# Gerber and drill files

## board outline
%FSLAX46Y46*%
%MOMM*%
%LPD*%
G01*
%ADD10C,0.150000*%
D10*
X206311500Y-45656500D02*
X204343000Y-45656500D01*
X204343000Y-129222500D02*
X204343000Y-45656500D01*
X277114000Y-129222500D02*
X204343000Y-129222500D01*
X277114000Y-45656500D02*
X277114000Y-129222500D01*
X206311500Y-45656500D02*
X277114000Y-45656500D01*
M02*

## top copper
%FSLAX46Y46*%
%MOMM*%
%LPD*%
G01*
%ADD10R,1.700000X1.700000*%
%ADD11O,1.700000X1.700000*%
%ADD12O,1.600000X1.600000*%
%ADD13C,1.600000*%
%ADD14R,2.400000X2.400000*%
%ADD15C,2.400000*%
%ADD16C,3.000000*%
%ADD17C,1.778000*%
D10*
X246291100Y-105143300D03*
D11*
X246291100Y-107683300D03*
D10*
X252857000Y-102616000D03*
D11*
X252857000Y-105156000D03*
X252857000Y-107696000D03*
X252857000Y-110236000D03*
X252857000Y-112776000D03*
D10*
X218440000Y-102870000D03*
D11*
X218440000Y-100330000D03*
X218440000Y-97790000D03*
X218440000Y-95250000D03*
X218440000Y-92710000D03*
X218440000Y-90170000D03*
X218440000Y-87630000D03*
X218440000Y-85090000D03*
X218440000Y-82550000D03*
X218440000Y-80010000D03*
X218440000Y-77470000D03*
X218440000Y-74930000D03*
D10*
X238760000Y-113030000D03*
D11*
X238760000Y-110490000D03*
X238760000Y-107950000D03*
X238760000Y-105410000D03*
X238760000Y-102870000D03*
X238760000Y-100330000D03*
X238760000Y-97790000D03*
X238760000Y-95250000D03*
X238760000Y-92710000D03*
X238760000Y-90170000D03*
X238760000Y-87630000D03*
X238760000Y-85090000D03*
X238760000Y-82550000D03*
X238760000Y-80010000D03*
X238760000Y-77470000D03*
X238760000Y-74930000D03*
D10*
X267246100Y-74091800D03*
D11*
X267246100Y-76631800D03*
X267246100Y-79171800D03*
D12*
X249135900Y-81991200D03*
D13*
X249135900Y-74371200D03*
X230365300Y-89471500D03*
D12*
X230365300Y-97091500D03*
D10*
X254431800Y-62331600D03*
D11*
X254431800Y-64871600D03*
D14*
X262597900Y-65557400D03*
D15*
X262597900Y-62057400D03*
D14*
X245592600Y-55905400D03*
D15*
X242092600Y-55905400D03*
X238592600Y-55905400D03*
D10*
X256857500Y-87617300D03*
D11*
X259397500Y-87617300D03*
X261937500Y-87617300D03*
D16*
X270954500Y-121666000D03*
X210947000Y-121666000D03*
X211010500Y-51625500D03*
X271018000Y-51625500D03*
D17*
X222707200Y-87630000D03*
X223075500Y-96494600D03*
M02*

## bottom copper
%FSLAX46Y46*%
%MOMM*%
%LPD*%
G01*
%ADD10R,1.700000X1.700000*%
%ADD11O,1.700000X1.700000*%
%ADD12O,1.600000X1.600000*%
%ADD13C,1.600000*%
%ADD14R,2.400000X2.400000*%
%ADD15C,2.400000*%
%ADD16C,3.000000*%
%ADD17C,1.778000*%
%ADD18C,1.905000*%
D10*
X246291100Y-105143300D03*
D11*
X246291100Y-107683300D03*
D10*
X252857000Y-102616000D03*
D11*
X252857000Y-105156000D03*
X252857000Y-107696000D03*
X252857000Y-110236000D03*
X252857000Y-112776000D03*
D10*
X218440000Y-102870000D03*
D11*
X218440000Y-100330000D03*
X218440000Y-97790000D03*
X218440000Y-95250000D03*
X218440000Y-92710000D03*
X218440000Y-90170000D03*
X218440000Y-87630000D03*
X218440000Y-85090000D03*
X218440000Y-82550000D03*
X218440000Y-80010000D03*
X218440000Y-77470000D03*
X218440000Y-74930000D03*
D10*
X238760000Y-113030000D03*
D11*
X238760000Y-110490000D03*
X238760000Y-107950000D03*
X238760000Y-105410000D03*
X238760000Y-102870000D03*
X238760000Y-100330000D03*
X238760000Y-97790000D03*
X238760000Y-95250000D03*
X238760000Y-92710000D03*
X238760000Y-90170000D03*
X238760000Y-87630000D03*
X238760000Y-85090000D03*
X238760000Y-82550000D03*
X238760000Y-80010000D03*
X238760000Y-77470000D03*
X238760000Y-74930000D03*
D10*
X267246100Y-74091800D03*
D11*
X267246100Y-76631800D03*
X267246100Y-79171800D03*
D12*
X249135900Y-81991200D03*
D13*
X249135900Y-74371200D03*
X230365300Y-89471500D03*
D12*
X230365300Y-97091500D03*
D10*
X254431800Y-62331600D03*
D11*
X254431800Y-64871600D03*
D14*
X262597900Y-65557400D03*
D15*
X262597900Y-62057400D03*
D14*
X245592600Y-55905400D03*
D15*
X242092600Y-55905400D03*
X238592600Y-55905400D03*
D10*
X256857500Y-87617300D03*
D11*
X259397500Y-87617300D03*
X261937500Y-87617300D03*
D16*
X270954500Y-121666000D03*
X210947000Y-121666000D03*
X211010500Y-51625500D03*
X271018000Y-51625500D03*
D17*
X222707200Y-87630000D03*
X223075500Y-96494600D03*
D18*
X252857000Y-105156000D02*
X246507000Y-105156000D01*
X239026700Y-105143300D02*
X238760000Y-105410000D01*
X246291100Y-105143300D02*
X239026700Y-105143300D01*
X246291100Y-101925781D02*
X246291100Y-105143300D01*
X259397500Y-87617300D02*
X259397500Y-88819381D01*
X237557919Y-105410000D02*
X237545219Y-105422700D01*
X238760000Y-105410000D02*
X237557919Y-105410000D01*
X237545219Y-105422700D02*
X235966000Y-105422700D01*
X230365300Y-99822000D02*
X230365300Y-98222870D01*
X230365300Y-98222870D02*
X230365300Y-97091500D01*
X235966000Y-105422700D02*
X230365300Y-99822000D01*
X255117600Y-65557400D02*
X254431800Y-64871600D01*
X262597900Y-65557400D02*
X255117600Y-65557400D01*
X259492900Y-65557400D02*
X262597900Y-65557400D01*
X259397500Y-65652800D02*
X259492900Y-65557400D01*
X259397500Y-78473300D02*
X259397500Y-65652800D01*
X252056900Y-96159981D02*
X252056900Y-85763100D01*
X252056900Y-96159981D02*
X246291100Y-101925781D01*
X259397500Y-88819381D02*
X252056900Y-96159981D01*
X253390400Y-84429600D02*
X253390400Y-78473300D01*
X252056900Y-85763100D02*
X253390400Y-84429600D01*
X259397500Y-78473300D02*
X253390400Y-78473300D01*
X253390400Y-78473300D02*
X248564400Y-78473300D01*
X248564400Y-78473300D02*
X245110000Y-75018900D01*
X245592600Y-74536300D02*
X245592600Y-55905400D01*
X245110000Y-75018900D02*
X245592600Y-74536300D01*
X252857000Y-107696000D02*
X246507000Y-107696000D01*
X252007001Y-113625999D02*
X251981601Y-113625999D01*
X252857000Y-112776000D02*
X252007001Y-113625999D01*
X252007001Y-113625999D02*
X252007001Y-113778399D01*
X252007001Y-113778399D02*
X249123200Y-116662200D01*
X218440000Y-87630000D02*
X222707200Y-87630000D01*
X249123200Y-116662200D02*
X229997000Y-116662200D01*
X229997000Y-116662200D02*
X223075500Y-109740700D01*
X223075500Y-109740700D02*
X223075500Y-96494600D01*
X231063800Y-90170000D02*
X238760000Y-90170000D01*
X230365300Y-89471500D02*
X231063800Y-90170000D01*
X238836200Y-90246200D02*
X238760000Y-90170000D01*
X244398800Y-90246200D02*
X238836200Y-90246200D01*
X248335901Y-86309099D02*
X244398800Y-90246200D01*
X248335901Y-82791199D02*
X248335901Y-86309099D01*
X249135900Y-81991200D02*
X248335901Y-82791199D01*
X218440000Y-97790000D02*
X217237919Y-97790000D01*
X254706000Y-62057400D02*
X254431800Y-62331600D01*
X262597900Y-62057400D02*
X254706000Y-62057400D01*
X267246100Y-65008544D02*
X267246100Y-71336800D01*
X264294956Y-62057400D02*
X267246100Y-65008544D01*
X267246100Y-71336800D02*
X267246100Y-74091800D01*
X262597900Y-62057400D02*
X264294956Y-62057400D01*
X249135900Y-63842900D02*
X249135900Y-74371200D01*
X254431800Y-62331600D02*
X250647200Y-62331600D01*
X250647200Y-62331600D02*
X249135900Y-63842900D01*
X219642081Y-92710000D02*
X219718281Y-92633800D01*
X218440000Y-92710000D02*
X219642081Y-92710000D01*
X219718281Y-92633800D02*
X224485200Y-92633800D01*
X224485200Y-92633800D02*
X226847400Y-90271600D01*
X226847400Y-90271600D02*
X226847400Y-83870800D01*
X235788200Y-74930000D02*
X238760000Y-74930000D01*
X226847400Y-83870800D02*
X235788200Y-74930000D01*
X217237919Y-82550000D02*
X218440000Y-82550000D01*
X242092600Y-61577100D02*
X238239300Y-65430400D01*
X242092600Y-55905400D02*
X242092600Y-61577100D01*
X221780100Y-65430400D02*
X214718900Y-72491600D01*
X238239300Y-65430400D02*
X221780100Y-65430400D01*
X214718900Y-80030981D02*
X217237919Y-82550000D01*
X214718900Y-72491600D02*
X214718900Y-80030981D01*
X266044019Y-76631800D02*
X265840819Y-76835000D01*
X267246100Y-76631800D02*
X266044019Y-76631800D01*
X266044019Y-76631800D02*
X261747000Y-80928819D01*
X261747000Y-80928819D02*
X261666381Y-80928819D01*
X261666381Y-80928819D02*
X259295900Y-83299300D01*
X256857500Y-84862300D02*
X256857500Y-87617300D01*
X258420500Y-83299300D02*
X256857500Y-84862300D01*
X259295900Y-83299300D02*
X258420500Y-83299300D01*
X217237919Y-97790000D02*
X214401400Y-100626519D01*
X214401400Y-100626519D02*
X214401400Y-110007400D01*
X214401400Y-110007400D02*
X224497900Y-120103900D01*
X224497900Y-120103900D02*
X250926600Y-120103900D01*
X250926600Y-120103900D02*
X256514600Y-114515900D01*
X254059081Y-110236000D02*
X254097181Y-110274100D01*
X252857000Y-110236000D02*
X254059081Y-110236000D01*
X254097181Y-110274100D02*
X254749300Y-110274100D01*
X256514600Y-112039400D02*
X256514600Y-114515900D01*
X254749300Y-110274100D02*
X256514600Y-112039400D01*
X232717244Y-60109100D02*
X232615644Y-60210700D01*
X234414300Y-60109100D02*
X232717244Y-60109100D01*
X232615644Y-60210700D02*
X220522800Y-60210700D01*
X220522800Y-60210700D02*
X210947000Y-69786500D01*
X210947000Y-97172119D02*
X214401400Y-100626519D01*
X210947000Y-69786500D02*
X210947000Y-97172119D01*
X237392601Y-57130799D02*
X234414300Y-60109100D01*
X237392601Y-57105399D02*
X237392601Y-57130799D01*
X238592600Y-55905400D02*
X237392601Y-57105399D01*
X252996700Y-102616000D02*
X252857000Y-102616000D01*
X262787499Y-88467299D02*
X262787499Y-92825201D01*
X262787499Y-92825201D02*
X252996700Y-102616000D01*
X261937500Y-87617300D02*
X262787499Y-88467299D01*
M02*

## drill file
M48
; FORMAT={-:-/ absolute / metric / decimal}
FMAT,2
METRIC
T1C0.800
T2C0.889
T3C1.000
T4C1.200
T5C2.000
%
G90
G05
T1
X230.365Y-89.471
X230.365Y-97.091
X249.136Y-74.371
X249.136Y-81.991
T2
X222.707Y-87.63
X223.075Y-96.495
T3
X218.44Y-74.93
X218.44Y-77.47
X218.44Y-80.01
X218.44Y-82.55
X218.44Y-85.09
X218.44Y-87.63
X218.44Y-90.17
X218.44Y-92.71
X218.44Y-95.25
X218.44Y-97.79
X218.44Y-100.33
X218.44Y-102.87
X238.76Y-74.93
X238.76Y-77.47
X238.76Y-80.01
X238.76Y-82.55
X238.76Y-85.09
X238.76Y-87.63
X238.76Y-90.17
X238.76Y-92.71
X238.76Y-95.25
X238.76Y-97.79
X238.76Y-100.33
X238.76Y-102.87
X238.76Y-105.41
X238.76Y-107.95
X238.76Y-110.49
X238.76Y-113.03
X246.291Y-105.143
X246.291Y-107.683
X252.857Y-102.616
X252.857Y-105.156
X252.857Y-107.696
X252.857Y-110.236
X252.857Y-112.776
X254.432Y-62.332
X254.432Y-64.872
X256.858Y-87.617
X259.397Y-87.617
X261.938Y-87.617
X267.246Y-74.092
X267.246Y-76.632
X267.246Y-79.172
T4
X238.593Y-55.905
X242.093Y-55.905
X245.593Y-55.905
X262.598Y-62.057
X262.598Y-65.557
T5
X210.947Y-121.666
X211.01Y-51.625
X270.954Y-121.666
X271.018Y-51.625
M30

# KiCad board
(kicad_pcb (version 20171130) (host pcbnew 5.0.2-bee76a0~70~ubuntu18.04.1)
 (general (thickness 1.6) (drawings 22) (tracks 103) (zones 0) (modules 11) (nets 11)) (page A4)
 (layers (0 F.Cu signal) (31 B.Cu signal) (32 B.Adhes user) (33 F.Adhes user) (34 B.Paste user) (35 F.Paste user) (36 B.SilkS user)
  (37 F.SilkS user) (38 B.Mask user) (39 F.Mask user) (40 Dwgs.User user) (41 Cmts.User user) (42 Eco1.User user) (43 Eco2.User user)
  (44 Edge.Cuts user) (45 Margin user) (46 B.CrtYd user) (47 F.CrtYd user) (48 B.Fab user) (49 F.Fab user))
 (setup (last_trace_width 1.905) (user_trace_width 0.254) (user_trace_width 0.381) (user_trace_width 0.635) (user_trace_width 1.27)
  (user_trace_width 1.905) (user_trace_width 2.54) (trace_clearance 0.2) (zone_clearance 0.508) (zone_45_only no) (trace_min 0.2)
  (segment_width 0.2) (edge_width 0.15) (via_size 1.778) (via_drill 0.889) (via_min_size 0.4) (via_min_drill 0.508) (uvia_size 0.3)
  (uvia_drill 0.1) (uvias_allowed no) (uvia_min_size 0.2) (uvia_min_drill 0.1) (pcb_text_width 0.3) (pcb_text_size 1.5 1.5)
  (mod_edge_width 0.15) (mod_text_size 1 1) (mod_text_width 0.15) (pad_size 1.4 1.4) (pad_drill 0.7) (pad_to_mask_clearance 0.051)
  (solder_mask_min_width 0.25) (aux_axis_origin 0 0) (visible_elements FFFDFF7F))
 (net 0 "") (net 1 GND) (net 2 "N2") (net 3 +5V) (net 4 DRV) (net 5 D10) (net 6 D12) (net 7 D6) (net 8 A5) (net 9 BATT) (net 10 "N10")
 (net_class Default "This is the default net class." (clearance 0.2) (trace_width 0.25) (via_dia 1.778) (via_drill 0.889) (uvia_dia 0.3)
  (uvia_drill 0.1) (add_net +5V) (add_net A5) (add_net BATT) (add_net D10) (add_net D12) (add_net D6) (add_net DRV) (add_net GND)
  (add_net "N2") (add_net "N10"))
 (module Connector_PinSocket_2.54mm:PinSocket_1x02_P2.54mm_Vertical (layer F.Cu) (at 246.2911 105.1433)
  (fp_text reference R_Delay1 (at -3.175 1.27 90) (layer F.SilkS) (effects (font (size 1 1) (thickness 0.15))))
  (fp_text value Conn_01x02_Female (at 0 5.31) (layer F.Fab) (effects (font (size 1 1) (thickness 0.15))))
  (pad 1 thru_hole rect (at 0 0) (size 1.7 1.7) (drill 1) (layers *.Cu *.Mask) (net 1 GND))
  (pad 2 thru_hole oval (at 0 2.54) (size 1.7 1.7) (drill 1) (layers *.Cu *.Mask) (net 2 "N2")))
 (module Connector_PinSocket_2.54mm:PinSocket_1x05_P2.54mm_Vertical (layer F.Cu) (at 252.857 102.616)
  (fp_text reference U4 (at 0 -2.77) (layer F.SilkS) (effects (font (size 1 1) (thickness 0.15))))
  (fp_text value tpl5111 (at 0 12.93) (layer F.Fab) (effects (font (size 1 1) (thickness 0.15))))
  (pad 1 thru_hole rect (at 0 0) (size 1.7 1.7) (drill 1) (layers *.Cu *.Mask) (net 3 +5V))
  (pad 2 thru_hole oval (at 0 2.54) (size 1.7 1.7) (drill 1) (layers *.Cu *.Mask) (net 1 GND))
  (pad 3 thru_hole oval (at 0 5.08) (size 1.7 1.7) (drill 1) (layers *.Cu *.Mask) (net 2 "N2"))
  (pad 4 thru_hole oval (at 0 7.62) (size 1.7 1.7) (drill 1) (layers *.Cu *.Mask) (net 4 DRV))
  (pad 5 thru_hole oval (at 0 10.16) (size 1.7 1.7) (drill 1) (layers *.Cu *.Mask) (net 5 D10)))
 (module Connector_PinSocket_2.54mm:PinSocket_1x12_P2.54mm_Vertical (layer F.Cu) (at 218.44 102.87 180)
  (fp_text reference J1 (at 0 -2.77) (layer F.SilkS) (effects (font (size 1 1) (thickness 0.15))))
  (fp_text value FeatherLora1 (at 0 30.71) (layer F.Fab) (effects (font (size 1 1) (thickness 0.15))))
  (pad 1 thru_hole rect (at 0 0 180) (size 1.7 1.7) (drill 1) (layers *.Cu *.Mask))
  (pad 2 thru_hole oval (at 0 2.54 180) (size 1.7 1.7) (drill 1) (layers *.Cu *.Mask))
  (pad 3 thru_hole oval (at 0 5.08 180) (size 1.7 1.7) (drill 1) (layers *.Cu *.Mask) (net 4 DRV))
  (pad 4 thru_hole oval (at 0 7.62 180) (size 1.7 1.7) (drill 1) (layers *.Cu *.Mask))
  (pad 5 thru_hole oval (at 0 10.16 180) (size 1.7 1.7) (drill 1) (layers *.Cu *.Mask) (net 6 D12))
  (pad 6 thru_hole oval (at 0 12.7 180) (size 1.7 1.7) (drill 1) (layers *.Cu *.Mask))
  (pad 7 thru_hole oval (at 0 15.24 180) (size 1.7 1.7) (drill 1) (layers *.Cu *.Mask) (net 5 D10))
  (pad 8 thru_hole oval (at 0 17.78 180) (size 1.7 1.7) (drill 1) (layers *.Cu *.Mask))
  (pad 9 thru_hole oval (at 0 20.32 180) (size 1.7 1.7) (drill 1) (layers *.Cu *.Mask) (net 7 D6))
  (pad 10 thru_hole oval (at 0 22.86 180) (size 1.7 1.7) (drill 1) (layers *.Cu *.Mask))
  (pad 11 thru_hole oval (at 0 25.4 180) (size 1.7 1.7) (drill 1) (layers *.Cu *.Mask))
  (pad 12 thru_hole oval (at 0 27.94 180) (size 1.7 1.7) (drill 1) (layers *.Cu *.Mask)))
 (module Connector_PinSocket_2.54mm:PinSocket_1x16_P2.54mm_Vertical (layer F.Cu) (at 238.76 113.03 180)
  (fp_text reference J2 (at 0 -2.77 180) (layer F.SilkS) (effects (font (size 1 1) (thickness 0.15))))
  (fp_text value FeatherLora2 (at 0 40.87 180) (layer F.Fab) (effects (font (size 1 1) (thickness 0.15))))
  (pad 1 thru_hole rect (at 0 0 180) (size 1.7 1.7) (drill 1) (layers *.Cu *.Mask))
  (pad 2 thru_hole oval (at 0 2.54 180) (size 1.7 1.7) (drill 1) (layers *.Cu *.Mask))
  (pad 3 thru_hole oval (at 0 5.08 180) (size 1.7 1.7) (drill 1) (layers *.Cu *.Mask))
  (pad 4 thru_hole oval (at 0 7.62 180) (size 1.7 1.7) (drill 1) (layers *.Cu *.Mask) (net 1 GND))
  (pad 5 thru_hole oval (at 0 10.16 180) (size 1.7 1.7) (drill 1) (layers *.Cu *.Mask))
  (pad 6 thru_hole oval (at 0 12.7 180) (size 1.7 1.7) (drill 1) (layers *.Cu *.Mask))
  (pad 7 thru_hole oval (at 0 15.24 180) (size 1.7 1.7) (drill 1) (layers *.Cu *.Mask))
  (pad 8 thru_hole oval (at 0 17.78 180) (size 1.7 1.7) (drill 1) (layers *.Cu *.Mask))
  (pad 9 thru_hole oval (at 0 20.32 180) (size 1.7 1.7) (drill 1) (layers *.Cu *.Mask))
  (pad 10 thru_hole oval (at 0 22.86 180) (size 1.7 1.7) (drill 1) (layers *.Cu *.Mask) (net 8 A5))
  (pad 11 thru_hole oval (at 0 25.4 180) (size 1.7 1.7) (drill 1) (layers *.Cu *.Mask))
  (pad 12 thru_hole oval (at 0 27.94 180) (size 1.7 1.7) (drill 1) (layers *.Cu *.Mask))
  (pad 13 thru_hole oval (at 0 30.48 180) (size 1.7 1.7) (drill 1) (layers *.Cu *.Mask))
  (pad 14 thru_hole oval (at 0 33.02 180) (size 1.7 1.7) (drill 1) (layers *.Cu *.Mask))
  (pad 15 thru_hole oval (at 0 35.56 180) (size 1.7 1.7) (drill 1) (layers *.Cu *.Mask))
  (pad 16 thru_hole oval (at 0 38.1 180) (size 1.7 1.7) (drill 1) (layers *.Cu *.Mask) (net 6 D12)))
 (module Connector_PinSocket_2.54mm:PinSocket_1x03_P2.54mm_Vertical (layer F.Cu) (at 267.2461 74.0918)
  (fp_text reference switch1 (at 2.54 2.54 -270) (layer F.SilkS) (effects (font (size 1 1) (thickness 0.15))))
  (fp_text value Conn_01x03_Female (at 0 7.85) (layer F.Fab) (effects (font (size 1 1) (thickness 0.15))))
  (pad 1 thru_hole rect (at 0 0) (size 1.7 1.7) (drill 1) (layers *.Cu *.Mask) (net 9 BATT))
  (pad 2 thru_hole oval (at 0 2.54) (size 1.7 1.7) (drill 1) (layers *.Cu *.Mask) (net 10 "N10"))
  (pad 3 thru_hole oval (at 0 5.08) (size 1.7 1.7) (drill 1) (layers *.Cu *.Mask)))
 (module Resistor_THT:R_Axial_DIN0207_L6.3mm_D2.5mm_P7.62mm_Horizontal (layer F.Cu) (at 249.1359 74.3712 270)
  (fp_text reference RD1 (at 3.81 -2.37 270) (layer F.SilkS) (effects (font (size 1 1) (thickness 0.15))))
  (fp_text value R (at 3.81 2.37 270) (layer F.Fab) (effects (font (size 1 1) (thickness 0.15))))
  (pad 2 thru_hole oval (at 7.62 0 270) (size 1.6 1.6) (drill 0.8) (layers *.Cu *.Mask) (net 8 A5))
  (pad 1 thru_hole circle (at 0 0 270) (size 1.6 1.6) (drill 0.8) (layers *.Cu *.Mask) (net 9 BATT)))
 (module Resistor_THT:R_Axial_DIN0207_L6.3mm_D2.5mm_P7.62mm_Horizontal (layer F.Cu) (at 230.3653 89.4715 270)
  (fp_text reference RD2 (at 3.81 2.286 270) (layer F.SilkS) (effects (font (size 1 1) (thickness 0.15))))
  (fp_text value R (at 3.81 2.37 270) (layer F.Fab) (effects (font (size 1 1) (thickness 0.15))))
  (pad 1 thru_hole circle (at 0 0 270) (size 1.6 1.6) (drill 0.8) (layers *.Cu *.Mask) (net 8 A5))
  (pad 2 thru_hole oval (at 7.62 0 270) (size 1.6 1.6) (drill 0.8) (layers *.Cu *.Mask) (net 1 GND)))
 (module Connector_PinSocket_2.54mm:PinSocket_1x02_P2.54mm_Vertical (layer F.Cu) (at 254.4318 62.3316)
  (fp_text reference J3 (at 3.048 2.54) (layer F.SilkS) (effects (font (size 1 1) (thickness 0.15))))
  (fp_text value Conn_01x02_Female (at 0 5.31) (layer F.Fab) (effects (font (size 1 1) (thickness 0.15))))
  (pad 1 thru_hole rect (at 0 0) (size 1.7 1.7) (drill 1) (layers *.Cu *.Mask) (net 9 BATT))
  (pad 2 thru_hole oval (at 0 2.54) (size 1.7 1.7) (drill 1) (layers *.Cu *.Mask) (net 1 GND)))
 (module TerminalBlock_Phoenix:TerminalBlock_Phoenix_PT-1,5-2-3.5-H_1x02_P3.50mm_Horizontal (layer F.Cu) (at 262.5979 65.5574 90)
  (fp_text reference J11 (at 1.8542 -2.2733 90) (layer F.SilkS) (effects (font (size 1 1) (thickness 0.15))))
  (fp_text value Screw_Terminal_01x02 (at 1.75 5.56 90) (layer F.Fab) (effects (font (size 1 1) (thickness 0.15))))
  (pad 1 thru_hole rect (at 0 0 90) (size 2.4 2.4) (drill 1.2) (layers *.Cu *.Mask) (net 1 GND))
  (pad 2 thru_hole circle (at 3.5 0 90) (size 2.4 2.4) (drill 1.2) (layers *.Cu *.Mask) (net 9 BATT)))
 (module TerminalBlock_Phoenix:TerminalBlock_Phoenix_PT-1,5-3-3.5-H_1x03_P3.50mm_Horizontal (layer F.Cu) (at 245.5926 55.9054 180)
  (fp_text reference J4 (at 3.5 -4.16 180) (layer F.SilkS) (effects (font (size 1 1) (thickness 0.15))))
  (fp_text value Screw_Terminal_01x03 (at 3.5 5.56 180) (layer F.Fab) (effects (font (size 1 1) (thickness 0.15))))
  (pad 1 thru_hole rect (at 0 0 180) (size 2.4 2.4) (drill 1.2) (layers *.Cu *.Mask) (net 1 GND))
  (pad 2 thru_hole circle (at 3.5 0 180) (size 2.4 2.4) (drill 1.2) (layers *.Cu *.Mask) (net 7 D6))
  (pad 3 thru_hole circle (at 7 0 180) (size 2.4 2.4) (drill 1.2) (layers *.Cu *.Mask) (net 4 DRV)))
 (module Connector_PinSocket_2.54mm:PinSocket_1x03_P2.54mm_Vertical (layer F.Cu) (at 256.8575 87.6173 90)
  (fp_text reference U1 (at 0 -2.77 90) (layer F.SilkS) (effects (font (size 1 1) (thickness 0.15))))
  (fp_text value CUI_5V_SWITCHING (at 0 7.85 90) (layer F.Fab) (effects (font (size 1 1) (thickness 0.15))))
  (pad 1 thru_hole rect (at 0 0 90) (size 1.7 1.7) (drill 1) (layers *.Cu *.Mask) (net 10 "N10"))
  (pad 2 thru_hole oval (at 0 2.54 90) (size 1.7 1.7) (drill 1) (layers *.Cu *.Mask) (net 1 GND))
  (pad 3 thru_hole oval (at 0 5.08 90) (size 1.7 1.7) (drill 1) (layers *.Cu *.Mask) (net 3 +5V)))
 (gr_line (start 206.3115 45.6565) (end 204.343 45.6565) (layer Edge.Cuts) (width 0.15))
 (gr_line (start 204.343 129.2225) (end 204.343 45.6565) (layer Edge.Cuts) (width 0.15))
 (gr_line (start 277.114 129.2225) (end 204.343 129.2225) (layer Edge.Cuts) (width 0.15))
 (gr_line (start 277.114 45.6565) (end 277.114 129.2225) (layer Edge.Cuts) (width 0.15))
 (gr_line (start 206.3115 45.6565) (end 277.114 45.6565) (layer Edge.Cuts) (width 0.15))
 (via (at 270.9545 121.666) (size 3) (drill 2) (layers F.Cu B.Cu) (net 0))
 (via (at 210.947 121.666) (size 3) (drill 2) (layers F.Cu B.Cu) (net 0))
 (via (at 211.0105 51.6255) (size 3) (drill 2) (layers F.Cu B.Cu) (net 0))
 (via (at 271.018 51.6255) (size 3) (drill 2) (layers F.Cu B.Cu) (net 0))
 (segment (start 252.857 105.156) (end 246.507 105.156) (width 1.905) (layer B.Cu) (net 1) (status 30))
 (segment (start 239.0267 105.1433) (end 238.76 105.41) (width 1.905) (layer B.Cu) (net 1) (status 30))
 (segment (start 246.2911 105.1433) (end 239.0267 105.1433) (width 1.905) (layer B.Cu) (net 1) (status 30))
 (segment (start 246.2911 101.925781) (end 246.2911 105.1433) (width 1.905) (layer B.Cu) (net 1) (status 20))
 (segment (start 259.3975 87.6173) (end 259.3975 88.819381) (width 1.905) (layer B.Cu) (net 1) (status 10))
 (segment (start 237.557919 105.41) (end 237.545219 105.4227) (width 1.905) (layer B.Cu) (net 1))
 (segment (start 238.76 105.41) (end 237.557919 105.41) (width 1.905) (layer B.Cu) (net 1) (status 10))
 (segment (start 237.545219 105.4227) (end 235.966 105.4227) (width 1.905) (layer B.Cu) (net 1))
 (segment (start 230.3653 99.822) (end 230.3653 98.22287) (width 1.905) (layer B.Cu) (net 1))
 (segment (start 230.3653 98.22287) (end 230.3653 97.0915) (width 1.905) (layer B.Cu) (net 1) (status 20))
 (segment (start 235.966 105.4227) (end 230.3653 99.822) (width 1.905) (layer B.Cu) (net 1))
 (segment (start 255.1176 65.5574) (end 254.4318 64.8716) (width 1.905) (layer B.Cu) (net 1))
 (segment (start 262.5979 65.5574) (end 255.1176 65.5574) (width 1.905) (layer B.Cu) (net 1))
 (segment (start 259.4929 65.5574) (end 262.5979 65.5574) (width 1.905) (layer B.Cu) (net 1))
 (segment (start 259.3975 65.6528) (end 259.4929 65.5574) (width 1.905) (layer B.Cu) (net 1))
 (segment (start 259.3975 78.4733) (end 259.3975 65.6528) (width 1.905) (layer B.Cu) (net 1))
 (segment (start 252.0569 96.159981) (end 252.0569 85.7631) (width 1.905) (layer B.Cu) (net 1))
 (segment (start 252.0569 96.159981) (end 246.2911 101.925781) (width 1.905) (layer B.Cu) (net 1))
 (segment (start 259.3975 88.819381) (end 252.0569 96.159981) (width 1.905) (layer B.Cu) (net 1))
 (segment (start 253.3904 84.4296) (end 253.3904 78.4733) (width 1.905) (layer B.Cu) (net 1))
 (segment (start 252.0569 85.7631) (end 253.3904 84.4296) (width 1.905) (layer B.Cu) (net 1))
 (segment (start 259.3975 78.4733) (end 253.3904 78.4733) (width 1.905) (layer B.Cu) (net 1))
 (segment (start 253.3904 78.4733) (end 248.5644 78.4733) (width 1.905) (layer B.Cu) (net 1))
 (segment (start 248.5644 78.4733) (end 245.11 75.0189) (width 1.905) (layer B.Cu) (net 1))
 (segment (start 245.5926 74.5363) (end 245.5926 55.9054) (width 1.905) (layer B.Cu) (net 1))
 (segment (start 245.11 75.0189) (end 245.5926 74.5363) (width 1.905) (layer B.Cu) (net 1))
 (segment (start 252.857 107.696) (end 246.507 107.696) (width 1.905) (layer B.Cu) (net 2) (status 30))
 (segment (start 252.007001 113.625999) (end 251.981601 113.625999) (width 1.905) (layer B.Cu) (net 5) (status 10))
 (segment (start 252.857 112.776) (end 252.007001 113.625999) (width 1.905) (layer B.Cu) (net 5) (status 30))
 (segment (start 252.007001 113.625999) (end 252.007001 113.778399) (width 1.905) (layer B.Cu) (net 5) (status 10))
 (segment (start 252.007001 113.778399) (end 249.1232 116.6622) (width 1.905) (layer B.Cu) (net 5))
 (segment (start 218.44 87.63) (end 222.7072 87.63) (width 1.905) (layer B.Cu) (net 5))
 (via (at 222.7072 87.63) (size 1.778) (drill 0.889) (layers F.Cu B.Cu) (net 5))
 (segment (start 249.1232 116.6622) (end 229.997 116.6622) (width 1.905) (layer B.Cu) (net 5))
 (via (at 223.0755 96.4946) (size 1.778) (drill 0.889) (layers F.Cu B.Cu) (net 5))
 (segment (start 229.997 116.6622) (end 223.0755 109.7407) (width 1.905) (layer B.Cu) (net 5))
 (segment (start 223.0755 109.7407) (end 223.0755 96.4946) (width 1.905) (layer B.Cu) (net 5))
 (segment (start 231.0638 90.17) (end 238.76 90.17) (width 1.905) (layer B.Cu) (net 8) (status 20))
 (segment (start 230.3653 89.4715) (end 231.0638 90.17) (width 1.905) (layer B.Cu) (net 8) (status 10))
 (segment (start 238.8362 90.2462) (end 238.76 90.17) (width 1.905) (layer B.Cu) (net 8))
 (segment (start 244.3988 90.2462) (end 238.8362 90.2462) (width 1.905) (layer B.Cu) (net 8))
 (segment (start 248.335901 86.309099) (end 244.3988 90.2462) (width 1.905) (layer B.Cu) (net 8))
 (segment (start 248.335901 82.791199) (end 248.335901 86.309099) (width 1.905) (layer B.Cu) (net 8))
 (segment (start 249.1359 81.9912) (end 248.335901 82.791199) (width 1.905) (layer B.Cu) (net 8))
 (segment (start 218.44 97.79) (end 217.237919 97.79) (width 1.905) (layer B.Cu) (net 4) (status 10))
 (segment (start 254.706 62.0574) (end 254.4318 62.3316) (width 1.905) (layer B.Cu) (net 9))
 (segment (start 262.5979 62.0574) (end 254.706 62.0574) (width 1.905) (layer B.Cu) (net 9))
 (segment (start 267.2461 65.008544) (end 267.2461 71.3368) (width 1.905) (layer B.Cu) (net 9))
 (segment (start 264.294956 62.0574) (end 267.2461 65.008544) (width 1.905) (layer B.Cu) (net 9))
 (segment (start 267.2461 71.3368) (end 267.2461 74.0918) (width 1.905) (layer B.Cu) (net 9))
 (segment (start 262.5979 62.0574) (end 264.294956 62.0574) (width 1.905) (layer B.Cu) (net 9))
 (segment (start 249.1359 63.8429) (end 249.1359 74.3712) (width 1.905) (layer B.Cu) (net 9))
 (segment (start 254.4318 62.3316) (end 250.6472 62.3316) (width 1.905) (layer B.Cu) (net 9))
 (segment (start 250.6472 62.3316) (end 249.1359 63.8429) (width 1.905) (layer B.Cu) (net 9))
 (segment (start 219.642081 92.71) (end 219.718281 92.6338) (width 1.905) (layer B.Cu) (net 6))
 (segment (start 218.44 92.71) (end 219.642081 92.71) (width 1.905) (layer B.Cu) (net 6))
 (segment (start 219.718281 92.6338) (end 224.4852 92.6338) (width 1.905) (layer B.Cu) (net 6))
 (segment (start 224.4852 92.6338) (end 226.8474 90.2716) (width 1.905) (layer B.Cu) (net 6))
 (segment (start 226.8474 90.2716) (end 226.8474 83.8708) (width 1.905) (layer B.Cu) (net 6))
 (segment (start 235.7882 74.93) (end 238.76 74.93) (width 1.905) (layer B.Cu) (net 6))
 (segment (start 226.8474 83.8708) (end 235.7882 74.93) (width 1.905) (layer B.Cu) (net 6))
 (segment (start 217.237919 82.55) (end 218.44 82.55) (width 1.905) (layer B.Cu) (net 7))
 (segment (start 242.0926 61.5771) (end 238.2393 65.4304) (width 1.905) (layer B.Cu) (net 7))
 (segment (start 242.0926 55.9054) (end 242.0926 61.5771) (width 1.905) (layer B.Cu) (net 7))
 (segment (start 221.7801 65.4304) (end 214.7189 72.4916) (width 1.905) (layer B.Cu) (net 7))
 (segment (start 238.2393 65.4304) (end 221.7801 65.4304) (width 1.905) (layer B.Cu) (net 7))
 (segment (start 214.7189 80.030981) (end 217.237919 82.55) (width 1.905) (layer B.Cu) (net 7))
 (segment (start 214.7189 72.4916) (end 214.7189 80.030981) (width 1.905) (layer B.Cu) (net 7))
 (segment (start 266.044019 76.6318) (end 265.840819 76.835) (width 1.905) (layer B.Cu) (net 10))
 (segment (start 267.2461 76.6318) (end 266.044019 76.6318) (width 1.905) (layer B.Cu) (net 10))
 (segment (start 266.044019 76.6318) (end 261.747 80.928819) (width 1.905) (layer B.Cu) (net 10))
 (segment (start 261.747 80.928819) (end 261.666381 80.928819) (width 1.905) (layer B.Cu) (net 10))
 (segment (start 261.666381 80.928819) (end 259.2959 83.2993) (width 1.905) (layer B.Cu) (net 10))
 (segment (start 256.8575 84.8623) (end 256.8575 87.6173) (width 1.905) (layer B.Cu) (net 10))
 (segment (start 258.4205 83.2993) (end 256.8575 84.8623) (width 1.905) (layer B.Cu) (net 10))
 (segment (start 259.2959 83.2993) (end 258.4205 83.2993) (width 1.905) (layer B.Cu) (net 10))
 (segment (start 217.237919 97.79) (end 214.4014 100.626519) (width 1.905) (layer B.Cu) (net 4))
 (segment (start 214.4014 100.626519) (end 214.4014 110.0074) (width 1.905) (layer B.Cu) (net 4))
 (segment (start 214.4014 110.0074) (end 224.4979 120.1039) (width 1.905) (layer B.Cu) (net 4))
 (segment (start 224.4979 120.1039) (end 250.9266 120.1039) (width 1.905) (layer B.Cu) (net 4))
 (segment (start 250.9266 120.1039) (end 256.5146 114.5159) (width 1.905) (layer B.Cu) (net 4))
 (segment (start 254.059081 110.236) (end 254.097181 110.2741) (width 1.905) (layer B.Cu) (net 4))
 (segment (start 252.857 110.236) (end 254.059081 110.236) (width 1.905) (layer B.Cu) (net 4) (status 10))
 (segment (start 254.097181 110.2741) (end 254.7493 110.2741) (width 1.905) (layer B.Cu) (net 4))
 (segment (start 256.5146 112.0394) (end 256.5146 114.5159) (width 1.905) (layer B.Cu) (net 4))
 (segment (start 254.7493 110.2741) (end 256.5146 112.0394) (width 1.905) (layer B.Cu) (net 4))
 (segment (start 232.717244 60.1091) (end 232.615644 60.2107) (width 1.905) (layer B.Cu) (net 4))
 (segment (start 234.4143 60.1091) (end 232.717244 60.1091) (width 1.905) (layer B.Cu) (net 4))
 (segment (start 232.615644 60.2107) (end 220.5228 60.2107) (width 1.905) (layer B.Cu) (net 4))
 (segment (start 220.5228 60.2107) (end 210.947 69.7865) (width 1.905) (layer B.Cu) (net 4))
 (segment (start 210.947 97.172119) (end 214.4014 100.626519) (width 1.905) (layer B.Cu) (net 4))
 (segment (start 210.947 69.7865) (end 210.947 97.172119) (width 1.905) (layer B.Cu) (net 4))
 (segment (start 237.392601 57.130799) (end 234.4143 60.1091) (width 1.905) (layer B.Cu) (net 4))
 (segment (start 237.392601 57.105399) (end 237.392601 57.130799) (width 1.905) (layer B.Cu) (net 4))
 (segment (start 238.5926 55.9054) (end 237.392601 57.105399) (width 1.905) (layer B.Cu) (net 4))
 (segment (start 252.9967 102.616) (end 252.857 102.616) (width 1.905) (layer B.Cu) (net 3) (status 30))
 (segment (start 262.787499 88.467299) (end 262.787499 92.825201) (width 1.905) (layer B.Cu) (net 3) (status 10))
 (segment (start 262.787499 92.825201) (end 252.9967 102.616) (width 1.905) (layer B.Cu) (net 3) (status 20))
 (segment (start 261.9375 87.6173) (end 262.787499 88.467299) (width 1.905) (layer B.Cu) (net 3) (status 30)))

